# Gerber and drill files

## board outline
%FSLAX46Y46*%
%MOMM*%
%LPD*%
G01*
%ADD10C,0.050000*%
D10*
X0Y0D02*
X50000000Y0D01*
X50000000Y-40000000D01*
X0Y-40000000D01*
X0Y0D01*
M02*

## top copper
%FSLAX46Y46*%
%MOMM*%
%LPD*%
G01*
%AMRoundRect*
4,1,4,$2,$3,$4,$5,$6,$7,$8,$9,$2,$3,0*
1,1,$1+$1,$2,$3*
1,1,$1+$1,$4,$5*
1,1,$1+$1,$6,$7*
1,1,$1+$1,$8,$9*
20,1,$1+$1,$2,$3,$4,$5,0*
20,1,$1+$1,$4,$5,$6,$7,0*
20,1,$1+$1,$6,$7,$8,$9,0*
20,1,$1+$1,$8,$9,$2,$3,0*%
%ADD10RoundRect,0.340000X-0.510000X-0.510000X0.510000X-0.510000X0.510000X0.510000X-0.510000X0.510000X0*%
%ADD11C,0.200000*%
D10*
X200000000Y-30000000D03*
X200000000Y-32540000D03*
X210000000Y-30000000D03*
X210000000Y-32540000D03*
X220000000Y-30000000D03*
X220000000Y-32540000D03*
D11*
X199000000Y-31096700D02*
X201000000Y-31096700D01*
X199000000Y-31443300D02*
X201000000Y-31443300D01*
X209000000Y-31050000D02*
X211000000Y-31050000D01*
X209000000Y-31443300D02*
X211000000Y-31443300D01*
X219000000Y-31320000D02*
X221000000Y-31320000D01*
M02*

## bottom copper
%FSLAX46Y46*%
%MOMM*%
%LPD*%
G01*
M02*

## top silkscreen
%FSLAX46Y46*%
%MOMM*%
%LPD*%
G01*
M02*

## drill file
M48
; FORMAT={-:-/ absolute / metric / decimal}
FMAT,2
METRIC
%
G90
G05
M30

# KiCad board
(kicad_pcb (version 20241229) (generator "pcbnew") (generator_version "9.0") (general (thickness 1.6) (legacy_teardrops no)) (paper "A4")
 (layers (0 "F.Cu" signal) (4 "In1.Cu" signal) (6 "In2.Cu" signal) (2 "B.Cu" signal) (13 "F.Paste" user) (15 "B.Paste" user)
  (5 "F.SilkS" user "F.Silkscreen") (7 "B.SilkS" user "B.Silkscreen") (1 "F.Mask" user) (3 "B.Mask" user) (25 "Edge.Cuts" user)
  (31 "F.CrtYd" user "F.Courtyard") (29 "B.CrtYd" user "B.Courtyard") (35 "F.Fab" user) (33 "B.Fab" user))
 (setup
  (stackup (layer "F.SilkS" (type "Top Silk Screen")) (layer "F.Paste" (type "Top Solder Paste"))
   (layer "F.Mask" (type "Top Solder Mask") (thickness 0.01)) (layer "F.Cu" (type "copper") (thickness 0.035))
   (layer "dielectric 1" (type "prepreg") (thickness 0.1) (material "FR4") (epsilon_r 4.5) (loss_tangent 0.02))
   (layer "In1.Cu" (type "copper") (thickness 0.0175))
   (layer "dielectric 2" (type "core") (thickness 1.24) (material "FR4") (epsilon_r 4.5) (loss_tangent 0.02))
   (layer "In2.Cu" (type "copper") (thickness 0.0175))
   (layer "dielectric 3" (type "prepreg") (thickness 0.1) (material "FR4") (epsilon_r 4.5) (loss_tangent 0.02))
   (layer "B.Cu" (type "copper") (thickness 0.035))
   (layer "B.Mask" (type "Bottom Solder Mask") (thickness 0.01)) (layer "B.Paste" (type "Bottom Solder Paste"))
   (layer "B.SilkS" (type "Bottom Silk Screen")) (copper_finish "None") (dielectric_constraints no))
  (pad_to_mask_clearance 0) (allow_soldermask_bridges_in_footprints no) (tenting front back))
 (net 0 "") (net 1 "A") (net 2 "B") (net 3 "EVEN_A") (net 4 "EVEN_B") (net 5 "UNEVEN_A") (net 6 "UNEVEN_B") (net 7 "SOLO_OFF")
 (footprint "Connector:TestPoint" (layer "F.Cu") (at 200 30)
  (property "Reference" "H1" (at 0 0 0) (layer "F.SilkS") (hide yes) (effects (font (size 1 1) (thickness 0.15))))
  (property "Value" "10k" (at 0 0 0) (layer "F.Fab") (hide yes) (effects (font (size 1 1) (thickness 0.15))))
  (pad "1" smd roundrect (at 0 0) (size 1.7 1.7) (layers "F.Cu" "F.Paste" "F.Mask") (roundrect_rratio 0.2) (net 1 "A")))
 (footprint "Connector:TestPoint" (layer "F.Cu") (at 200 32.54)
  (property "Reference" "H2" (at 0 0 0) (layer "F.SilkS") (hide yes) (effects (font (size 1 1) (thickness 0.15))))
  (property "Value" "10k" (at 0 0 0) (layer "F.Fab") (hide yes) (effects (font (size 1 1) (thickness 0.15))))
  (pad "1" smd roundrect (at 0 0) (size 1.7 1.7) (layers "F.Cu" "F.Paste" "F.Mask") (roundrect_rratio 0.2) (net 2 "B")))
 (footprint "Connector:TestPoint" (layer "F.Cu") (at 210 30)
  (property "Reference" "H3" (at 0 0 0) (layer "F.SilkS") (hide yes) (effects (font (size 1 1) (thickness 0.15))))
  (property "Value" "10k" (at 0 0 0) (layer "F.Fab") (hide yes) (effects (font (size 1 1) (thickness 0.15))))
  (pad "1" smd roundrect (at 0 0) (size 1.7 1.7) (layers "F.Cu" "F.Paste" "F.Mask") (roundrect_rratio 0.2) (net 1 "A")))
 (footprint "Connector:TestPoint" (layer "F.Cu") (at 210 32.54)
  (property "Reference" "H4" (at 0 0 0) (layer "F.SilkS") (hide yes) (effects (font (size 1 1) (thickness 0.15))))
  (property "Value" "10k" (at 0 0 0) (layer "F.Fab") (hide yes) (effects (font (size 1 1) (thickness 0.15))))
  (pad "1" smd roundrect (at 0 0) (size 1.7 1.7) (layers "F.Cu" "F.Paste" "F.Mask") (roundrect_rratio 0.2) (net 2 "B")))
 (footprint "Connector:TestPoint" (layer "F.Cu") (at 220 30)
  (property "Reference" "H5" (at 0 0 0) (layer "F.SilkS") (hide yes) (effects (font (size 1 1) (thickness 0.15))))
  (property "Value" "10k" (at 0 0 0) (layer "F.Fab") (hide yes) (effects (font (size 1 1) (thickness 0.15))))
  (pad "1" smd roundrect (at 0 0) (size 1.7 1.7) (layers "F.Cu" "F.Paste" "F.Mask") (roundrect_rratio 0.2) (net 1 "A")))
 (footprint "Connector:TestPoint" (layer "F.Cu") (at 220 32.54)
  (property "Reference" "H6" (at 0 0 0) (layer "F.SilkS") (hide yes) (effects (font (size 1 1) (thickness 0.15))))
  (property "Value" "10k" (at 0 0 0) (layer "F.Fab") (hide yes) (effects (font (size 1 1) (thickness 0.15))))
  (pad "1" smd roundrect (at 0 0) (size 1.7 1.7) (layers "F.Cu" "F.Paste" "F.Mask") (roundrect_rratio 0.2) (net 2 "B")))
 (segment (start 199 31.0967) (end 201 31.0967) (width 0.2) (layer "F.Cu") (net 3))
 (segment (start 199 31.4433) (end 201 31.4433) (width 0.2) (layer "F.Cu") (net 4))
 (segment (start 209 31.05) (end 211 31.05) (width 0.2) (layer "F.Cu") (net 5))
 (segment (start 209 31.4433) (end 211 31.4433) (width 0.2) (layer "F.Cu") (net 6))
 (segment (start 219 31.32) (end 221 31.32) (width 0.2) (layer "F.Cu") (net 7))
 (gr_rect (start 0 0) (end 50 40) (stroke (width 0.05) (type default)) (fill no) (layer "Edge.Cuts")))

